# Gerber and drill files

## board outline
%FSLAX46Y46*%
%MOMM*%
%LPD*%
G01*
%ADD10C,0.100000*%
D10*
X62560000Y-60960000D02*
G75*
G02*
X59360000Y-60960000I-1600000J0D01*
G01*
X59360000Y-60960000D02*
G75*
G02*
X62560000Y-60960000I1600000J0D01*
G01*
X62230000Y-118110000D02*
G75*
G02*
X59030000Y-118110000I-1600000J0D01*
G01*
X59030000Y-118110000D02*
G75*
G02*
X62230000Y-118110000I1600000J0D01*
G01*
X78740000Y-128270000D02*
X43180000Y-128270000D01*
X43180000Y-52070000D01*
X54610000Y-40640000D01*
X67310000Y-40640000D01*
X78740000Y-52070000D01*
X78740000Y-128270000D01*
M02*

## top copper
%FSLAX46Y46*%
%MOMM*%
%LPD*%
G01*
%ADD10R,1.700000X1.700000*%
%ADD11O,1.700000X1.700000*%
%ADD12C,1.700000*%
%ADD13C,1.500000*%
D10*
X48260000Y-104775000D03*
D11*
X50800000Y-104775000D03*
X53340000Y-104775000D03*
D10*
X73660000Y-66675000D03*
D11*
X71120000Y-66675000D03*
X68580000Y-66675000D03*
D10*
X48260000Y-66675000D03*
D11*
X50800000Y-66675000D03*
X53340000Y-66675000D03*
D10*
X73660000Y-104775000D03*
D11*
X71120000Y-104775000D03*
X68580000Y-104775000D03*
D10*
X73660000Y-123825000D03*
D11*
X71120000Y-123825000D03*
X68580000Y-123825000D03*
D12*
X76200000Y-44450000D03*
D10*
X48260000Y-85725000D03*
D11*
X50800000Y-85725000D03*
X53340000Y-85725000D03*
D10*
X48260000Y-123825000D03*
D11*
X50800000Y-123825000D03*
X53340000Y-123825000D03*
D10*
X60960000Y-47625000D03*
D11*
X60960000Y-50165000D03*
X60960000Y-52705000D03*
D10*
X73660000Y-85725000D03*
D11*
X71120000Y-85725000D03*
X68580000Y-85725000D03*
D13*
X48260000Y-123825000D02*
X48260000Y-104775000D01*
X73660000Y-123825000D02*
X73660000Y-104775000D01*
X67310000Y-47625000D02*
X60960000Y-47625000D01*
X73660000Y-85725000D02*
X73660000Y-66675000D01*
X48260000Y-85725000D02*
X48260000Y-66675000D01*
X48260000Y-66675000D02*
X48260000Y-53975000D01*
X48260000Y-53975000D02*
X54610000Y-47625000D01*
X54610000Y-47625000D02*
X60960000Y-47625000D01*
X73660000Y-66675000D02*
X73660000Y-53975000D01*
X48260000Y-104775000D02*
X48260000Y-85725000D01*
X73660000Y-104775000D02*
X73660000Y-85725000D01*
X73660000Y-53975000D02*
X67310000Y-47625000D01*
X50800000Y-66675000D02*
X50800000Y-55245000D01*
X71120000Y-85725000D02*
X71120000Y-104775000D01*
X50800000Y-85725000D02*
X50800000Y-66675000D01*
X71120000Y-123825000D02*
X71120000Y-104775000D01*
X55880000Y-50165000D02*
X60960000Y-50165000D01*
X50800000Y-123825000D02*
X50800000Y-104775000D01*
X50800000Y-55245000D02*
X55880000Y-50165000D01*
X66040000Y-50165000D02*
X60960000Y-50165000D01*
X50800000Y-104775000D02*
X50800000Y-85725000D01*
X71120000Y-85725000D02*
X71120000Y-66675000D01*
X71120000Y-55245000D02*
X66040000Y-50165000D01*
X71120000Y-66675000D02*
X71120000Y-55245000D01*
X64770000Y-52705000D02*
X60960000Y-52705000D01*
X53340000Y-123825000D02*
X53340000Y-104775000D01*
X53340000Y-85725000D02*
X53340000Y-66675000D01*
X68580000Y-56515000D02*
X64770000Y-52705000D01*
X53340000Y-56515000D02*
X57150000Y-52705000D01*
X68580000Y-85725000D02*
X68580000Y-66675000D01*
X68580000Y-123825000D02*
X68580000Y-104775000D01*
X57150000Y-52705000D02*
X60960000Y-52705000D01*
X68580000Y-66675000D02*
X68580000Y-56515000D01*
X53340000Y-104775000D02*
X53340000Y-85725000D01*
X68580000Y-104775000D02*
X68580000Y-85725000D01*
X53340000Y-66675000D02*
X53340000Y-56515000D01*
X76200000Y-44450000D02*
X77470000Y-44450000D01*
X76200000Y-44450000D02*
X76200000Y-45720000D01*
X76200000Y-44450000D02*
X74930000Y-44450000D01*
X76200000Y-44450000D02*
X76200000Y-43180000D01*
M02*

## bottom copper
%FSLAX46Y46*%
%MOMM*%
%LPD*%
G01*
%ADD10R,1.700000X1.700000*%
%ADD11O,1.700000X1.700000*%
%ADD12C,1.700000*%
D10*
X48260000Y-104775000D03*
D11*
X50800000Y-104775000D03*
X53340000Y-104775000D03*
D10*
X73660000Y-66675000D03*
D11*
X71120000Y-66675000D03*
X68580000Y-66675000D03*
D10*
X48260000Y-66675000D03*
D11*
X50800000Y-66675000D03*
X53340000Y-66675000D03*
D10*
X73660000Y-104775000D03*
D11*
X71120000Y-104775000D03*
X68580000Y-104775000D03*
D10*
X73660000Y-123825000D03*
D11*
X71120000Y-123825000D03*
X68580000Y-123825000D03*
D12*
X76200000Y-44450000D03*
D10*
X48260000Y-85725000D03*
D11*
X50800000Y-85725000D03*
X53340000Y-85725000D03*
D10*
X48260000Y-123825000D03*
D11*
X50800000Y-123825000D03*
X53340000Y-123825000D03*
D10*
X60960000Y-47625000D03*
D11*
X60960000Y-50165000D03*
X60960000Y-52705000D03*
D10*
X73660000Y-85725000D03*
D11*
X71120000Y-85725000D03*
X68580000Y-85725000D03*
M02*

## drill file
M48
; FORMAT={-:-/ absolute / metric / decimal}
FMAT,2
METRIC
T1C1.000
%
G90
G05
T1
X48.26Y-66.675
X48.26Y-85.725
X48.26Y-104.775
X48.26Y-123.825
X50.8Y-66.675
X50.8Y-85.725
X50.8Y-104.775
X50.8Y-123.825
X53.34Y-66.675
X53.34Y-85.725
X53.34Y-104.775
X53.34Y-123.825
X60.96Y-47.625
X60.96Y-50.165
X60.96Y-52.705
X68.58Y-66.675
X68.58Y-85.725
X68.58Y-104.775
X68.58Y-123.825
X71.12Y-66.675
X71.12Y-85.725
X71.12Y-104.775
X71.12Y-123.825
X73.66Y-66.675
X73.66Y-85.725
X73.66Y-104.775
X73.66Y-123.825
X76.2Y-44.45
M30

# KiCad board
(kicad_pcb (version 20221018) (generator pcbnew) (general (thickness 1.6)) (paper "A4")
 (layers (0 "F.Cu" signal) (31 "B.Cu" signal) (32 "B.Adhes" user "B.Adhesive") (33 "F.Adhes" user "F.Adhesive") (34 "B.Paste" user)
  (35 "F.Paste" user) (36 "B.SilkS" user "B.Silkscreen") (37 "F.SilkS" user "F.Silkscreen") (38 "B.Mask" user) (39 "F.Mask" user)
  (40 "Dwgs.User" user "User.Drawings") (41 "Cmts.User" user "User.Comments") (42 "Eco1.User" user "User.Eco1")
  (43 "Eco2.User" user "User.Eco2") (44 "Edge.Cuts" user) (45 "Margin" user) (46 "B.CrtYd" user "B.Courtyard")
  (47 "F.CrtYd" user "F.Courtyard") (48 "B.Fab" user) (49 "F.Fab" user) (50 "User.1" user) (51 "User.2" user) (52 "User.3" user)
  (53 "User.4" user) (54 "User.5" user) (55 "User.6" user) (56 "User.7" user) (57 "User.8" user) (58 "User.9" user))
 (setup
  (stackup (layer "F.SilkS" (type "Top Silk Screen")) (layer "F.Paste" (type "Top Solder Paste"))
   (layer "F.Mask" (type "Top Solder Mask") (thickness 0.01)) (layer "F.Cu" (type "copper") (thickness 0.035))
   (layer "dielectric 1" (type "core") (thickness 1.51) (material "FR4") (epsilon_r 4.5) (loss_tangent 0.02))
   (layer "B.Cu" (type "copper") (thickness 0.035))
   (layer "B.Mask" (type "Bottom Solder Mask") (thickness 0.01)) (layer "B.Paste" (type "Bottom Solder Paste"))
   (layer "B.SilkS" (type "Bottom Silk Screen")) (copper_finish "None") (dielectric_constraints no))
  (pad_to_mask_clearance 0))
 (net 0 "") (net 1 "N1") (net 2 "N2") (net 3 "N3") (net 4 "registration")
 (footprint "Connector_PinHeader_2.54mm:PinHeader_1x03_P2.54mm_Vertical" (layer "F.Cu") (at 48.26 104.775 90)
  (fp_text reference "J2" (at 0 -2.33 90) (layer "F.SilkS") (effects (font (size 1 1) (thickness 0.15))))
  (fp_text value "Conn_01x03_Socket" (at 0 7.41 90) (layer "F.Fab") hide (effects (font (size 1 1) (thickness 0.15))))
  (pad "1" thru_hole rect (at 0 0 90) (size 1.7 1.7) (drill 1) (layers "*.Cu" "*.Mask") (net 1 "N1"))
  (pad "2" thru_hole oval (at 0 2.54 90) (size 1.7 1.7) (drill 1) (layers "*.Cu" "*.Mask") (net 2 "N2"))
  (pad "3" thru_hole oval (at 0 5.08 90) (size 1.7 1.7) (drill 1) (layers "*.Cu" "*.Mask") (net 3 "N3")))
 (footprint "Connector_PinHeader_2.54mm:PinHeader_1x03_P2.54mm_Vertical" (layer "F.Cu") (at 73.66 66.675 -90)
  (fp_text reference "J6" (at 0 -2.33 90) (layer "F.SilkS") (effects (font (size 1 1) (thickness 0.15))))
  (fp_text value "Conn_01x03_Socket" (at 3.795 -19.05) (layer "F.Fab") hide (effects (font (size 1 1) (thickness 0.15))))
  (pad "1" thru_hole rect (at 0 0 270) (size 1.7 1.7) (drill 1) (layers "*.Cu" "*.Mask") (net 1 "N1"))
  (pad "2" thru_hole oval (at 0 2.54 270) (size 1.7 1.7) (drill 1) (layers "*.Cu" "*.Mask") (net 2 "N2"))
  (pad "3" thru_hole oval (at 0 5.08 270) (size 1.7 1.7) (drill 1) (layers "*.Cu" "*.Mask") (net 3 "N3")))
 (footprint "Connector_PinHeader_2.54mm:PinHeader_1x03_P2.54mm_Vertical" (layer "F.Cu") (at 48.26 66.675 90)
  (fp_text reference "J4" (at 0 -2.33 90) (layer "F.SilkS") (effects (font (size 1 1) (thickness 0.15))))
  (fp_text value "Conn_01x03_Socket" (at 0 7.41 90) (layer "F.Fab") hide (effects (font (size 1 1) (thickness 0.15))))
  (pad "1" thru_hole rect (at 0 0 90) (size 1.7 1.7) (drill 1) (layers "*.Cu" "*.Mask") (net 1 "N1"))
  (pad "2" thru_hole oval (at 0 2.54 90) (size 1.7 1.7) (drill 1) (layers "*.Cu" "*.Mask") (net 2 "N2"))
  (pad "3" thru_hole oval (at 0 5.08 90) (size 1.7 1.7) (drill 1) (layers "*.Cu" "*.Mask") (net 3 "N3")))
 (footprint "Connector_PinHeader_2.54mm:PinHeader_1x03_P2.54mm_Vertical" (layer "F.Cu") (at 73.66 104.775 -90)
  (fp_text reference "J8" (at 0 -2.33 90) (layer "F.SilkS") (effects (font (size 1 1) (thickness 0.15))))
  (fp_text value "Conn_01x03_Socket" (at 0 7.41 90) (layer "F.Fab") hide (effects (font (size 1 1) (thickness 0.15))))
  (pad "1" thru_hole rect (at 0 0 270) (size 1.7 1.7) (drill 1) (layers "*.Cu" "*.Mask") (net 1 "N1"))
  (pad "2" thru_hole oval (at 0 2.54 270) (size 1.7 1.7) (drill 1) (layers "*.Cu" "*.Mask") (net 2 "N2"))
  (pad "3" thru_hole oval (at 0 5.08 270) (size 1.7 1.7) (drill 1) (layers "*.Cu" "*.Mask") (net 3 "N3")))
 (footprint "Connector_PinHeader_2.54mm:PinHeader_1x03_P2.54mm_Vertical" (layer "F.Cu") (at 73.66 123.825 -90)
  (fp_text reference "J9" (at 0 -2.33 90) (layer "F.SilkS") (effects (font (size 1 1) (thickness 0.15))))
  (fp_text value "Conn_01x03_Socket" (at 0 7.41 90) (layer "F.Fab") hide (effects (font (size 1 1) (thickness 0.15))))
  (pad "1" thru_hole rect (at 0 0 270) (size 1.7 1.7) (drill 1) (layers "*.Cu" "*.Mask") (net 1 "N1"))
  (pad "2" thru_hole oval (at 0 2.54 270) (size 1.7 1.7) (drill 1) (layers "*.Cu" "*.Mask") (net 2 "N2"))
  (pad "3" thru_hole oval (at 0 5.08 270) (size 1.7 1.7) (drill 1) (layers "*.Cu" "*.Mask") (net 3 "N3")))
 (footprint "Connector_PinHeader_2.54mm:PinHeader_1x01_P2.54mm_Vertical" (layer "F.Cu") (at 76.2 44.45)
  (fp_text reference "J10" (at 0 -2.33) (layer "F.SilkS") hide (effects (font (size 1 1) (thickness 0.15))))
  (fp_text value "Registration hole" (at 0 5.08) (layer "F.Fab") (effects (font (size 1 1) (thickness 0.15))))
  (pad "1" thru_hole circle (at 0 0) (size 1.7 1.7) (drill 1) (layers "*.Cu" "*.Mask") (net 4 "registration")))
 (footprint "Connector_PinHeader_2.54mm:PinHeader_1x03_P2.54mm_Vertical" (layer "F.Cu") (at 48.26 85.725 90)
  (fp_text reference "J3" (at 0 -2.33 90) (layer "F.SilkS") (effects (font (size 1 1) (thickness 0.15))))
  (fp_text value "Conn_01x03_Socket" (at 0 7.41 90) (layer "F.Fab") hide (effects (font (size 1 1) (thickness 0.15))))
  (pad "1" thru_hole rect (at 0 0 90) (size 1.7 1.7) (drill 1) (layers "*.Cu" "*.Mask") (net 1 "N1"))
  (pad "2" thru_hole oval (at 0 2.54 90) (size 1.7 1.7) (drill 1) (layers "*.Cu" "*.Mask") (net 2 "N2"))
  (pad "3" thru_hole oval (at 0 5.08 90) (size 1.7 1.7) (drill 1) (layers "*.Cu" "*.Mask") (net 3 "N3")))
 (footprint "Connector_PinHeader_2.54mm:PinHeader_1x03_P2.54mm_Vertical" (layer "F.Cu") (at 48.26 123.825 90)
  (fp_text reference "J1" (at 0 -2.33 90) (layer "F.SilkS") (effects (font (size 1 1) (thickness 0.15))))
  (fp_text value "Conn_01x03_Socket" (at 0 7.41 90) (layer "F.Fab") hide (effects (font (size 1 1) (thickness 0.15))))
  (pad "1" thru_hole rect (at 0 0 90) (size 1.7 1.7) (drill 1) (layers "*.Cu" "*.Mask") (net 1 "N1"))
  (pad "2" thru_hole oval (at 0 2.54 90) (size 1.7 1.7) (drill 1) (layers "*.Cu" "*.Mask") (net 2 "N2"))
  (pad "3" thru_hole oval (at 0 5.08 90) (size 1.7 1.7) (drill 1) (layers "*.Cu" "*.Mask") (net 3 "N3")))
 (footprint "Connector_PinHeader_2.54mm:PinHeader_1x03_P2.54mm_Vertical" (layer "F.Cu") (at 60.96 47.625)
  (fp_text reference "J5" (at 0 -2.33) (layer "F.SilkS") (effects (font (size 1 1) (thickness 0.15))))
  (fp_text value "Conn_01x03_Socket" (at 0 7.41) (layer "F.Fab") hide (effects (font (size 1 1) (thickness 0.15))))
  (pad "1" thru_hole rect (at 0 0) (size 1.7 1.7) (drill 1) (layers "*.Cu" "*.Mask") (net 1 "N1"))
  (pad "2" thru_hole oval (at 0 2.54) (size 1.7 1.7) (drill 1) (layers "*.Cu" "*.Mask") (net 2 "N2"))
  (pad "3" thru_hole oval (at 0 5.08) (size 1.7 1.7) (drill 1) (layers "*.Cu" "*.Mask") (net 3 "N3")))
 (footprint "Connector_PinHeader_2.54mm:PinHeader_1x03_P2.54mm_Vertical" (layer "F.Cu") (at 73.66 85.725 -90)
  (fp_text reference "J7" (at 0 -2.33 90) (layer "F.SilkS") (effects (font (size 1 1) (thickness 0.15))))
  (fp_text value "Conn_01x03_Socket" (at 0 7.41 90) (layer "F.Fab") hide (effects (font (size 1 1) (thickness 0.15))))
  (pad "1" thru_hole rect (at 0 0 270) (size 1.7 1.7) (drill 1) (layers "*.Cu" "*.Mask") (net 1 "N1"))
  (pad "2" thru_hole oval (at 0 2.54 270) (size 1.7 1.7) (drill 1) (layers "*.Cu" "*.Mask") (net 2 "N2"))
  (pad "3" thru_hole oval (at 0 5.08 270) (size 1.7 1.7) (drill 1) (layers "*.Cu" "*.Mask") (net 3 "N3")))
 (gr_circle (center 60.96 60.96) (end 62.56 60.96) (stroke (width 0.1) (type default)) (fill none) (layer "Edge.Cuts"))
 (gr_circle (center 60.63 118.11) (end 62.23 118.11) (stroke (width 0.1) (type default)) (fill none) (layer "Edge.Cuts"))
 (gr_poly
  (pts (xy 78.74 128.27) (xy 43.18 128.27) (xy 43.18 52.07) (xy 54.61 40.64) (xy 67.31 40.64) (xy 78.74 52.07))
  (stroke (width 0.1) (type solid)) (fill none) (layer "Edge.Cuts"))
 (segment (start 48.26 123.825) (end 48.26 104.775) (width 1.5) (layer "F.Cu") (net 1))
 (segment (start 73.66 123.825) (end 73.66 104.775) (width 1.5) (layer "F.Cu") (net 1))
 (segment (start 67.31 47.625) (end 60.96 47.625) (width 1.5) (layer "F.Cu") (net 1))
 (segment (start 73.66 85.725) (end 73.66 66.675) (width 1.5) (layer "F.Cu") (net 1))
 (segment (start 48.26 85.725) (end 48.26 66.675) (width 1.5) (layer "F.Cu") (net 1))
 (segment (start 48.26 66.675) (end 48.26 53.975) (width 1.5) (layer "F.Cu") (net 1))
 (segment (start 48.26 53.975) (end 54.61 47.625) (width 1.5) (layer "F.Cu") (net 1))
 (segment (start 54.61 47.625) (end 60.96 47.625) (width 1.5) (layer "F.Cu") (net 1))
 (segment (start 73.66 66.675) (end 73.66 53.975) (width 1.5) (layer "F.Cu") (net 1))
 (segment (start 48.26 104.775) (end 48.26 85.725) (width 1.5) (layer "F.Cu") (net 1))
 (segment (start 73.66 104.775) (end 73.66 85.725) (width 1.5) (layer "F.Cu") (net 1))
 (segment (start 73.66 53.975) (end 67.31 47.625) (width 1.5) (layer "F.Cu") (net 1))
 (segment (start 50.8 66.675) (end 50.8 55.245) (width 1.5) (layer "F.Cu") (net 2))
 (segment (start 71.12 85.725) (end 71.12 104.775) (width 1.5) (layer "F.Cu") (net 2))
 (segment (start 50.8 85.725) (end 50.8 66.675) (width 1.5) (layer "F.Cu") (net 2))
 (segment (start 71.12 123.825) (end 71.12 104.775) (width 1.5) (layer "F.Cu") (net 2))
 (segment (start 55.88 50.165) (end 60.96 50.165) (width 1.5) (layer "F.Cu") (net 2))
 (segment (start 50.8 123.825) (end 50.8 104.775) (width 1.5) (layer "F.Cu") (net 2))
 (segment (start 50.8 55.245) (end 55.88 50.165) (width 1.5) (layer "F.Cu") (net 2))
 (segment (start 66.04 50.165) (end 60.96 50.165) (width 1.5) (layer "F.Cu") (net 2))
 (segment (start 50.8 104.775) (end 50.8 85.725) (width 1.5) (layer "F.Cu") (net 2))
 (segment (start 71.12 85.725) (end 71.12 66.675) (width 1.5) (layer "F.Cu") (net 2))
 (segment (start 71.12 55.245) (end 66.04 50.165) (width 1.5) (layer "F.Cu") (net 2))
 (segment (start 71.12 66.675) (end 71.12 55.245) (width 1.5) (layer "F.Cu") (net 2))
 (segment (start 64.77 52.705) (end 60.96 52.705) (width 1.5) (layer "F.Cu") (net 3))
 (segment (start 53.34 123.825) (end 53.34 104.775) (width 1.5) (layer "F.Cu") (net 3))
 (segment (start 53.34 85.725) (end 53.34 66.675) (width 1.5) (layer "F.Cu") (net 3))
 (segment (start 68.58 56.515) (end 64.77 52.705) (width 1.5) (layer "F.Cu") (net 3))
 (segment (start 53.34 56.515) (end 57.15 52.705) (width 1.5) (layer "F.Cu") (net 3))
 (segment (start 68.58 85.725) (end 68.58 66.675) (width 1.5) (layer "F.Cu") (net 3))
 (segment (start 68.58 123.825) (end 68.58 104.775) (width 1.5) (layer "F.Cu") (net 3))
 (segment (start 57.15 52.705) (end 60.96 52.705) (width 1.5) (layer "F.Cu") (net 3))
 (segment (start 68.58 66.675) (end 68.58 56.515) (width 1.5) (layer "F.Cu") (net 3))
 (segment (start 53.34 104.775) (end 53.34 85.725) (width 1.5) (layer "F.Cu") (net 3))
 (segment (start 68.58 104.775) (end 68.58 85.725) (width 1.5) (layer "F.Cu") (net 3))
 (segment (start 53.34 66.675) (end 53.34 56.515) (width 1.5) (layer "F.Cu") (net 3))
 (segment (start 76.2 44.45) (end 77.47 44.45) (width 1.5) (layer "F.Cu") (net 4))
 (segment (start 76.2 44.45) (end 76.2 45.72) (width 1.5) (layer "F.Cu") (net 4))
 (segment (start 76.2 44.45) (end 74.93 44.45) (width 1.5) (layer "F.Cu") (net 4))
 (segment (start 76.2 44.45) (end 76.2 43.18) (width 1.5) (layer "F.Cu") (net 4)))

